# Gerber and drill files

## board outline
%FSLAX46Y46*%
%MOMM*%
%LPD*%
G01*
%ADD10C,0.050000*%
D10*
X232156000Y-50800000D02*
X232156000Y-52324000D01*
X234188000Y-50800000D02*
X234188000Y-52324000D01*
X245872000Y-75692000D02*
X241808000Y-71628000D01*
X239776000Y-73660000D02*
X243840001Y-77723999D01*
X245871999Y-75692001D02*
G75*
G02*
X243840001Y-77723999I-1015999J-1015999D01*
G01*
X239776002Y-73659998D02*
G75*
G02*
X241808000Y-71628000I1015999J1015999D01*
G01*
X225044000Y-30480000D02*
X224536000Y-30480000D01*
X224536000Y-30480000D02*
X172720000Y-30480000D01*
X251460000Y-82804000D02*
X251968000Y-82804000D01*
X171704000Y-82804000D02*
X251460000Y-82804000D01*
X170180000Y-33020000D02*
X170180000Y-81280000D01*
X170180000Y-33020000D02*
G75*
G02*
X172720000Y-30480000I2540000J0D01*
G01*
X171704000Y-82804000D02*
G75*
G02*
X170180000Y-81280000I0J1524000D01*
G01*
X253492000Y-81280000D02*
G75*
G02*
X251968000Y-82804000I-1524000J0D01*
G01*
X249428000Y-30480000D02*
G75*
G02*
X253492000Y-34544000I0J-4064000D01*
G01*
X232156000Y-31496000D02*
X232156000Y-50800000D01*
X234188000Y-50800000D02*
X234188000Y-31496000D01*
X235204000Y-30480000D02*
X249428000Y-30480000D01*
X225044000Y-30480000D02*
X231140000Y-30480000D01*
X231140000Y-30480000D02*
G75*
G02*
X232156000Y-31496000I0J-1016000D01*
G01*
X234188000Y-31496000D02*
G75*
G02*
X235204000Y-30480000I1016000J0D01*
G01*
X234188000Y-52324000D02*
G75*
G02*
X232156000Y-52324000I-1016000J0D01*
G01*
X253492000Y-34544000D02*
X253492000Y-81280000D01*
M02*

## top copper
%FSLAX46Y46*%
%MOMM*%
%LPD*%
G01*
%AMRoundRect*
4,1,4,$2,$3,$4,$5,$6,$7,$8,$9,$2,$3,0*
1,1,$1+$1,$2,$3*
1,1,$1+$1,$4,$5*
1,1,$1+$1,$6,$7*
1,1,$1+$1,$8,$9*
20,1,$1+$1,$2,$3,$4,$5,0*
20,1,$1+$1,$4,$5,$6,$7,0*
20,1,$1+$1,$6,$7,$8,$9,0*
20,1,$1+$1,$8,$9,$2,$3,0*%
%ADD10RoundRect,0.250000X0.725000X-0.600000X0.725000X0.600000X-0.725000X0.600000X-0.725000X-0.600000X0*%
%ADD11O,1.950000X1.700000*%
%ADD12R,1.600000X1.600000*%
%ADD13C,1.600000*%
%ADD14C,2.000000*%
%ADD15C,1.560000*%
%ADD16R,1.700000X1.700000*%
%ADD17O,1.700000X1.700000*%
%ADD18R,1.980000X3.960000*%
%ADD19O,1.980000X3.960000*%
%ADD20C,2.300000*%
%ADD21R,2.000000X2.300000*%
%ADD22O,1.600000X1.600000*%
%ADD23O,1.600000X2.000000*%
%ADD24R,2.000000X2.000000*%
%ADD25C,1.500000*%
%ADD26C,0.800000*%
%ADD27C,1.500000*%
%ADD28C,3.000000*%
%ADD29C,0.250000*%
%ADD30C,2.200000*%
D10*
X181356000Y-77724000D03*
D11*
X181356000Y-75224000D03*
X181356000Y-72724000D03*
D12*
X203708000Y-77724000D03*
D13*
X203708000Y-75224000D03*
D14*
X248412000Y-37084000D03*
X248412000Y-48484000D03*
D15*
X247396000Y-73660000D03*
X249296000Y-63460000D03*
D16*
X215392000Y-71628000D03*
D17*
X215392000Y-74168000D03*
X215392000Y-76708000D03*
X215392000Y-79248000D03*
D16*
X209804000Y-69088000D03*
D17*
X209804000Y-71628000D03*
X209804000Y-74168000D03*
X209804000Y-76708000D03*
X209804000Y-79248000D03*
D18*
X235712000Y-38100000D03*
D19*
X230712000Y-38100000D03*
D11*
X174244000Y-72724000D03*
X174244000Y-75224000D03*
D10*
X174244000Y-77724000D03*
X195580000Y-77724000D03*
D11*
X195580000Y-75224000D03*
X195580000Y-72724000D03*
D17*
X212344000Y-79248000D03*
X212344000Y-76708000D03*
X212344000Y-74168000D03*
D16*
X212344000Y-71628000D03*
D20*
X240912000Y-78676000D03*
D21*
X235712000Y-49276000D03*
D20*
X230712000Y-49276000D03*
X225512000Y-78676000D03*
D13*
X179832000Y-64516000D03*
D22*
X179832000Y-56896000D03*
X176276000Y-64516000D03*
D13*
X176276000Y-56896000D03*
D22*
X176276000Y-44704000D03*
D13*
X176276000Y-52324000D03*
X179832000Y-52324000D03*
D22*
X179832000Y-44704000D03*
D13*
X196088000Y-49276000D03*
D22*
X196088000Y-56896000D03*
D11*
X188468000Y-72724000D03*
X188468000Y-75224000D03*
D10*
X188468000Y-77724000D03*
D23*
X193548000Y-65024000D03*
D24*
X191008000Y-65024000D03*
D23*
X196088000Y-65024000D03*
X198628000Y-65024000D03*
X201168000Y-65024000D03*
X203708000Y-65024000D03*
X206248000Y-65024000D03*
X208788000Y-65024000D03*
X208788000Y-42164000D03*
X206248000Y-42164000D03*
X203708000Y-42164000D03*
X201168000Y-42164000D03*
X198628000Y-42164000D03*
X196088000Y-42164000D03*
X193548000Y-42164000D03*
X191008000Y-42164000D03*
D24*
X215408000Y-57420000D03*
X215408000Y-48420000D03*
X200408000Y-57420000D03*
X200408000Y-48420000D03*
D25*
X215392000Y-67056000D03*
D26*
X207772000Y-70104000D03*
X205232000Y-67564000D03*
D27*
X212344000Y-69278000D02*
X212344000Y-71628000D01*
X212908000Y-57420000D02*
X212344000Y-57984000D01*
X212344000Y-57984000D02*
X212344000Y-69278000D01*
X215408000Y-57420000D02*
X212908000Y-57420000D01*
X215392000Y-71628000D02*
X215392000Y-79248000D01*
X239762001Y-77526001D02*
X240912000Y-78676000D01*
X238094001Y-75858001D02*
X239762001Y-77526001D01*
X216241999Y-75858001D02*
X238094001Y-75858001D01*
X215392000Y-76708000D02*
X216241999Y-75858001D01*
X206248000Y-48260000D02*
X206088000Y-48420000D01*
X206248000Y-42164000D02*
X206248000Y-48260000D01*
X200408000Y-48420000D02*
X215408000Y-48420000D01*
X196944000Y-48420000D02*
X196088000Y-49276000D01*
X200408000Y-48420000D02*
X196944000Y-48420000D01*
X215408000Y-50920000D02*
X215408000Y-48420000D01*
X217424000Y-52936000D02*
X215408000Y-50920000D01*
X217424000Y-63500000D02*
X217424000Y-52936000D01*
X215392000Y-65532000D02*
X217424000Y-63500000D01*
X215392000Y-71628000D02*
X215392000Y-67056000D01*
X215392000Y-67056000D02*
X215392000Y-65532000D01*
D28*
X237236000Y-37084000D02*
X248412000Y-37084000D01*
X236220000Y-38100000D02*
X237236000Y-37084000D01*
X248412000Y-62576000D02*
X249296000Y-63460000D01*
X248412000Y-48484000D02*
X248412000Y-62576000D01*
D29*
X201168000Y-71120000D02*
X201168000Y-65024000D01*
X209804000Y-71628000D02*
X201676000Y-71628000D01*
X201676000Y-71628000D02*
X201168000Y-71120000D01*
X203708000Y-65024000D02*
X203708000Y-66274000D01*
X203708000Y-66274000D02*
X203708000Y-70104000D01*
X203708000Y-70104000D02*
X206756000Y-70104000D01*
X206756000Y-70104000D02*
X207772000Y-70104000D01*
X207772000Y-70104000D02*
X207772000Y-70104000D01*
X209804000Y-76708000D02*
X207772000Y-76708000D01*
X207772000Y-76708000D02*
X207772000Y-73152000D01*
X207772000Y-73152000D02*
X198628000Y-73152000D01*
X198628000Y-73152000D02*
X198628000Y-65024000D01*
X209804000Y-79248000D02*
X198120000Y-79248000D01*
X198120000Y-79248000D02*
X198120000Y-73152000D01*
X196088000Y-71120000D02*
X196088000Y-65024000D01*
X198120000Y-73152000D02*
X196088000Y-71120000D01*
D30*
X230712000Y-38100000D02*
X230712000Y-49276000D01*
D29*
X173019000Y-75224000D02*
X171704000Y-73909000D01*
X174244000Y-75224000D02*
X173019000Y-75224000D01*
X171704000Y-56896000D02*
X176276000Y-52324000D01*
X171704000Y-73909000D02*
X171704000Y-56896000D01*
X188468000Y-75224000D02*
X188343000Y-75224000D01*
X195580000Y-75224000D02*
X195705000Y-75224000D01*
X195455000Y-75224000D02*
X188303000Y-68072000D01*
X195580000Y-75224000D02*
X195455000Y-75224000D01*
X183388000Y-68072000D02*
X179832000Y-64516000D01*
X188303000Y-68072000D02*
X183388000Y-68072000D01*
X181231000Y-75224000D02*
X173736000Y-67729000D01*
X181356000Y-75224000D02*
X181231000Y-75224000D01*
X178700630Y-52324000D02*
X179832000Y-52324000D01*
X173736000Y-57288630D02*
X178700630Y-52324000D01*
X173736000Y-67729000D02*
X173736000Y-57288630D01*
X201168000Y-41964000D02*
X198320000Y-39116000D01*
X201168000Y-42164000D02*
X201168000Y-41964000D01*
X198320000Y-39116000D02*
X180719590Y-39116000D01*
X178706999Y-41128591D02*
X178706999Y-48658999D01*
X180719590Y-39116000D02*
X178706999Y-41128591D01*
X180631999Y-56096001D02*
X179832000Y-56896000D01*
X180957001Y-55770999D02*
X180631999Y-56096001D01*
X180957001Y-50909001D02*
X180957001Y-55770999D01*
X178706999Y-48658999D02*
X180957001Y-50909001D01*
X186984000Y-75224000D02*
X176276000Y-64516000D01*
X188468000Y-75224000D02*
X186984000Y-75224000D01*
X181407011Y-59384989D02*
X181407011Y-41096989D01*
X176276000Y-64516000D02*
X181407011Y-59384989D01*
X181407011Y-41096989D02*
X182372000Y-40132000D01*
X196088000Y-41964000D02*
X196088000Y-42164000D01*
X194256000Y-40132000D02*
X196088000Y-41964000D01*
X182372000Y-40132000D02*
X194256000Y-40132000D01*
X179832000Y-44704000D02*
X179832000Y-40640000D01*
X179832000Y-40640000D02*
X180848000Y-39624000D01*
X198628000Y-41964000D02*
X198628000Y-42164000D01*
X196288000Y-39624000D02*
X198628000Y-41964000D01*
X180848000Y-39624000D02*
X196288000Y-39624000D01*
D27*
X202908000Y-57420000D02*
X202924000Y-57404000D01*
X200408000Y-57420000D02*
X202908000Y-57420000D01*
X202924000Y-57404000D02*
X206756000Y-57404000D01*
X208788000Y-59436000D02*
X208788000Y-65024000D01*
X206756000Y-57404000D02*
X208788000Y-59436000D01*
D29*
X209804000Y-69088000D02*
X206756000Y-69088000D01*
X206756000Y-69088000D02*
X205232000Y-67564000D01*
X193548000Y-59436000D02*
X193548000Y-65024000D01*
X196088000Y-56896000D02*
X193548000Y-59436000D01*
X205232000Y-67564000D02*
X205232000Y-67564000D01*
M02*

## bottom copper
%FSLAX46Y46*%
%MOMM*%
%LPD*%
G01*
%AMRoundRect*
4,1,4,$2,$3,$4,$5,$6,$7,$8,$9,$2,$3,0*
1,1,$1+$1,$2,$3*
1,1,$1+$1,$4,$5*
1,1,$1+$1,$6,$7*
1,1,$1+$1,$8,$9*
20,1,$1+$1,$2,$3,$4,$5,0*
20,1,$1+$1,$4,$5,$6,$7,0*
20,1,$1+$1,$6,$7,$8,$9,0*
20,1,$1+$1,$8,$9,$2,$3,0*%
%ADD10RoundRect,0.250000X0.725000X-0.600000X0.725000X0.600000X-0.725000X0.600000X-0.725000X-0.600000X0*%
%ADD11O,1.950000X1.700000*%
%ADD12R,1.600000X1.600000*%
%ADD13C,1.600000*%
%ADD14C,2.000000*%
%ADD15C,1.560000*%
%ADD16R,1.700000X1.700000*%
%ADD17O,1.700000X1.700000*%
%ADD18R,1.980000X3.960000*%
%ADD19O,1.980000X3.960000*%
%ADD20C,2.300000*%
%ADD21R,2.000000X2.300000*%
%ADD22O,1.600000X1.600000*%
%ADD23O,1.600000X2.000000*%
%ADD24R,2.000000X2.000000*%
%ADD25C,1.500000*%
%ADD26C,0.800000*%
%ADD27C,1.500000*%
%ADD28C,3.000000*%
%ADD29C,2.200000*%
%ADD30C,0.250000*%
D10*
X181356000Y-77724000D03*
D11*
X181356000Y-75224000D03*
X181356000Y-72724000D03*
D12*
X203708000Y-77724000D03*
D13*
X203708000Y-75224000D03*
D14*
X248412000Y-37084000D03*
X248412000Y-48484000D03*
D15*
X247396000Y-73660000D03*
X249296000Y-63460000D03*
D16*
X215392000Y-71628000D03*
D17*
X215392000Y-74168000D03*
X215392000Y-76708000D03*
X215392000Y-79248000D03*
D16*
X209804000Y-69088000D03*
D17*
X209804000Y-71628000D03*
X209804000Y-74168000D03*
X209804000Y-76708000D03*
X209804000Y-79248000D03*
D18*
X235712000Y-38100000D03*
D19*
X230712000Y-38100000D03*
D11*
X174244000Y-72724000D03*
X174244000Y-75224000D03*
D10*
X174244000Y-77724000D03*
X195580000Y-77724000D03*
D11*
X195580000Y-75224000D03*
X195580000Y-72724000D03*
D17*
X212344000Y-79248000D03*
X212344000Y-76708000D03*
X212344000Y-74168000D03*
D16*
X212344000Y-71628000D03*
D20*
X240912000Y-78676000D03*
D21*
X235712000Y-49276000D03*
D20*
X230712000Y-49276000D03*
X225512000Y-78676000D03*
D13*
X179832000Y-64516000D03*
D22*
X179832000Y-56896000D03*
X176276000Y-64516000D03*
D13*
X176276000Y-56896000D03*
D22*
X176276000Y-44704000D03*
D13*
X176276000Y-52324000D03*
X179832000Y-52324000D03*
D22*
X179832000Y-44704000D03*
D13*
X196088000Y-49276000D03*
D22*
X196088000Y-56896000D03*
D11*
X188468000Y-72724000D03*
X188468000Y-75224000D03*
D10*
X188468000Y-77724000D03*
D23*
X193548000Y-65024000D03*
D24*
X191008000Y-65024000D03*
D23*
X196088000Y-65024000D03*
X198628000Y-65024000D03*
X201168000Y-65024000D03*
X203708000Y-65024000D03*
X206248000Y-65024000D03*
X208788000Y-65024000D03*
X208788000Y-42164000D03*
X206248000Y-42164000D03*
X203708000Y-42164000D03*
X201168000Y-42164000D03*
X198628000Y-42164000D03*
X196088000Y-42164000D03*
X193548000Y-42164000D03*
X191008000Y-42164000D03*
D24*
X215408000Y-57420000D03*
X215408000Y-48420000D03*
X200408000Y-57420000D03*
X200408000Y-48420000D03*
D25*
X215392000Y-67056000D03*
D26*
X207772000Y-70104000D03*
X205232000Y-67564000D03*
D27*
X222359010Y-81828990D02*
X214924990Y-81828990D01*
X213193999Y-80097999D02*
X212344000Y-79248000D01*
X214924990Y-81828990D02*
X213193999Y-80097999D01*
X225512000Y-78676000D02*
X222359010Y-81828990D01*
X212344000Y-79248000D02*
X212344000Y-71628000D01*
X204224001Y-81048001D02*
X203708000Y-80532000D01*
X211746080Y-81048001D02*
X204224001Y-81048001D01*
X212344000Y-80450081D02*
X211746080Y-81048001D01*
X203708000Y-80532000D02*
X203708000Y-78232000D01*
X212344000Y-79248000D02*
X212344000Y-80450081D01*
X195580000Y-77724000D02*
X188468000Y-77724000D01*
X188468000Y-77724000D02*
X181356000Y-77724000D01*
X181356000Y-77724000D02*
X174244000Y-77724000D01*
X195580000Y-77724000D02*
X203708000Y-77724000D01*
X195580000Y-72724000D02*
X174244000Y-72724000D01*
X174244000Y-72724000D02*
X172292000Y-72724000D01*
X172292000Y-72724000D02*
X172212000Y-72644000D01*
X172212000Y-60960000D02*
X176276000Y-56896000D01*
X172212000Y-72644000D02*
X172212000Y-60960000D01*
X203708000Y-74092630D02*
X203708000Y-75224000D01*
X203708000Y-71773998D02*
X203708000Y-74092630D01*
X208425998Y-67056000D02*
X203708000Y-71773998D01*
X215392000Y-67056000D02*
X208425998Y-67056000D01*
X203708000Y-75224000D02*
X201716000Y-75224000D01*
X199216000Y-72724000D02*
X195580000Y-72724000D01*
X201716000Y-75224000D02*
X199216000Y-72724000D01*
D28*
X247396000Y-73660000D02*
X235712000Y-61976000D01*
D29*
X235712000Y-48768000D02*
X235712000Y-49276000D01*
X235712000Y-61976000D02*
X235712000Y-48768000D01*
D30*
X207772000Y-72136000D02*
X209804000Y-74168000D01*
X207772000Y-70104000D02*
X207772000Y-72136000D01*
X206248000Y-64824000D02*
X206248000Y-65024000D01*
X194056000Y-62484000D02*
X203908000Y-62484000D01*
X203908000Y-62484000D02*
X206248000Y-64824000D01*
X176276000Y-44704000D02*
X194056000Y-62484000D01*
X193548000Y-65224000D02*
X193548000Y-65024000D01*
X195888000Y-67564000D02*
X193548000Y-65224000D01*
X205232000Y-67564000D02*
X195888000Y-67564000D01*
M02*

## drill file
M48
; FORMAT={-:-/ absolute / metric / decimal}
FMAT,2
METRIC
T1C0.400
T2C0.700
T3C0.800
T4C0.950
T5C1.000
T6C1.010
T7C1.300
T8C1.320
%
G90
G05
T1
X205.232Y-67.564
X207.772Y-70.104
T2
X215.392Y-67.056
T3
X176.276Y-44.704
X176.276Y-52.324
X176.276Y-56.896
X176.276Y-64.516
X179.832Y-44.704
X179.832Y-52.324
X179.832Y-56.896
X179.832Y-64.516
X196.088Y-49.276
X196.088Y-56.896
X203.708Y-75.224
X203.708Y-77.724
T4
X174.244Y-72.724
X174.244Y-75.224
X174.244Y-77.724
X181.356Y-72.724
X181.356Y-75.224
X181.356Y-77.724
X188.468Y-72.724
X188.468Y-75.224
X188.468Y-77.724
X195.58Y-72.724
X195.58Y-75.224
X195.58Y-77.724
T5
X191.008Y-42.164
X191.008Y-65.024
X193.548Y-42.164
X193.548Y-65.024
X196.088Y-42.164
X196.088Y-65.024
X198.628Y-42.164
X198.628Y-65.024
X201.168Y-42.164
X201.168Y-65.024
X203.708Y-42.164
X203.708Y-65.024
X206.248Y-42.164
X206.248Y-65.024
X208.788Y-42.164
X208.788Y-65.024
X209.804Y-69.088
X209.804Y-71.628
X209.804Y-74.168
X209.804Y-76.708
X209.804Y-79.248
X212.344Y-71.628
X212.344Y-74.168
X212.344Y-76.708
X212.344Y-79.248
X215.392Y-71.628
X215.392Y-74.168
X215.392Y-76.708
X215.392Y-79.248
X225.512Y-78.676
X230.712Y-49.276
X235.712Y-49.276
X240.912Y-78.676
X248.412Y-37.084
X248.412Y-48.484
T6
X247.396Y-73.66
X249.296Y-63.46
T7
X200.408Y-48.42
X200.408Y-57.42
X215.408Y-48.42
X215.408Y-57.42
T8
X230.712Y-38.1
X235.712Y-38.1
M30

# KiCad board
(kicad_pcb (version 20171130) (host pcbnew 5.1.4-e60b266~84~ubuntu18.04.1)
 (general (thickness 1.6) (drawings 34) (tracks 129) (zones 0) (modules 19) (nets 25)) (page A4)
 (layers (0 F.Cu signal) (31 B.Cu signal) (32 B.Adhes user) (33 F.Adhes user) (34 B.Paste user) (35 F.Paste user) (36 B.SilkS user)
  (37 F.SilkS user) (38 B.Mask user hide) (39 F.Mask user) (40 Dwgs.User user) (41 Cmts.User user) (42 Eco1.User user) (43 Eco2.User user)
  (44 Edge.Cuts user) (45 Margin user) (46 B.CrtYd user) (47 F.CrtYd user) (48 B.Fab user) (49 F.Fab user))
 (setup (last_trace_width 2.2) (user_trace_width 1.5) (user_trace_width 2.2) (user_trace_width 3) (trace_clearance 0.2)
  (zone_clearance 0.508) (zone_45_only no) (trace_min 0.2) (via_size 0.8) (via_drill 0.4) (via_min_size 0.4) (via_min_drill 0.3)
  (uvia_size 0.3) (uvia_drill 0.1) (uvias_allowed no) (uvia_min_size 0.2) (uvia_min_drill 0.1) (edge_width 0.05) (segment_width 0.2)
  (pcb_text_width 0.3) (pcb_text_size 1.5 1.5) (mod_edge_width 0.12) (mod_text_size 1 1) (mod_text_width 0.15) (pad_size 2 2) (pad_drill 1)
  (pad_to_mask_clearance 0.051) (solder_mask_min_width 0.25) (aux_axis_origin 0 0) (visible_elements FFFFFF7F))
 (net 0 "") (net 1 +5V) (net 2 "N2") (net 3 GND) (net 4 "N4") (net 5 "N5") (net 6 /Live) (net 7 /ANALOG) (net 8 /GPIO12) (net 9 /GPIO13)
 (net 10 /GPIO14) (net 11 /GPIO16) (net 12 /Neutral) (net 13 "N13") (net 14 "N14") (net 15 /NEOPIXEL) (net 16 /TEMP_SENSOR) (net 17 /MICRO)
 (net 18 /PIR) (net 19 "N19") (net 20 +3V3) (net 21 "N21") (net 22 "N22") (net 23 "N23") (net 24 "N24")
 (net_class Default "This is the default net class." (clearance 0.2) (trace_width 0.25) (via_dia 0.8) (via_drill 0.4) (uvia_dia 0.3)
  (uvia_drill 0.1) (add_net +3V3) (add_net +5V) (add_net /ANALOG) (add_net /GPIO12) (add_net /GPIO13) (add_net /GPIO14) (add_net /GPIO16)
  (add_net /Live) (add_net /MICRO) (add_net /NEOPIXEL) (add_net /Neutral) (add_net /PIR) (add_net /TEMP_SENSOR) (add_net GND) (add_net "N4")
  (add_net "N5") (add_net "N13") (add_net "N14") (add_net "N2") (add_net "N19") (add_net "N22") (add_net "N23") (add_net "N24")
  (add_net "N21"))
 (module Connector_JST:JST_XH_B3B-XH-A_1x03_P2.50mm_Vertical (layer F.Cu) (at 181.356 77.724 90)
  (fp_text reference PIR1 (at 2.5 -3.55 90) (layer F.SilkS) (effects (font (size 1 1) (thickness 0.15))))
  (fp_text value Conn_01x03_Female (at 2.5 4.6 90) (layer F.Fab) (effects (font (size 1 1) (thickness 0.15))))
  (pad 1 thru_hole roundrect (at 0 0 90) (size 1.7 1.95) (drill 0.95) (layers *.Cu *.Mask) (roundrect_rratio 0.147059) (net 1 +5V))
  (pad 2 thru_hole oval (at 2.5 0 90) (size 1.7 1.95) (drill 0.95) (layers *.Cu *.Mask) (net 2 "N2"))
  (pad 3 thru_hole oval (at 5 0 90) (size 1.7 1.95) (drill 0.95) (layers *.Cu *.Mask) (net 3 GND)))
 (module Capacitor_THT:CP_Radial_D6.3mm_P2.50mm (layer F.Cu) (at 203.708 77.724 90)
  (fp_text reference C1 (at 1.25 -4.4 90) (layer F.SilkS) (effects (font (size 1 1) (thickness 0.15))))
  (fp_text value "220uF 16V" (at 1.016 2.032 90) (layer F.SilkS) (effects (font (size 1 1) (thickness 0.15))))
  (pad 1 thru_hole rect (at 0 0 90) (size 1.6 1.6) (drill 0.8) (layers *.Cu *.Mask) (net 1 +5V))
  (pad 2 thru_hole circle (at 2.5 0 90) (size 1.6 1.6) (drill 0.8) (layers *.Cu *.Mask) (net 3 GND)))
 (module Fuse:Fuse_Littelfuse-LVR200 (layer F.Cu) (at 248.412 37.084 270)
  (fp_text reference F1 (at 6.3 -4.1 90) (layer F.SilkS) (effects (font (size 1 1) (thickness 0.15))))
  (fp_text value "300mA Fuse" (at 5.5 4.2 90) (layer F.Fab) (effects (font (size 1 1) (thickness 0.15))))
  (pad 1 thru_hole circle (at 0 0 270) (size 2 2) (drill 1) (layers *.Cu *.Mask) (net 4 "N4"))
  (pad 2 thru_hole circle (at 11.4 0 270) (size 2 2) (drill 1) (layers *.Cu *.Mask) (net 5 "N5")))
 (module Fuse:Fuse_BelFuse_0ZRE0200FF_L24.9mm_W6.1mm (layer F.Cu) (at 247.396 73.66 90)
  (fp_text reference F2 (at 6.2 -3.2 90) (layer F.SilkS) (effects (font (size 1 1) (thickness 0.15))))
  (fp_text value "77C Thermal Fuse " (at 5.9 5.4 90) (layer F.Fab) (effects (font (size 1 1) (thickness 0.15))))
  (pad 1 thru_hole circle (at 0 0 90) (size 1.56 1.56) (drill 1.01) (layers *.Cu *.Mask) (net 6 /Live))
  (pad 2 thru_hole circle (at 10.2 1.9 90) (size 1.56 1.56) (drill 1.01) (layers *.Cu *.Mask) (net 5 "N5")))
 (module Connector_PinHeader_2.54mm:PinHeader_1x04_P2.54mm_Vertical (layer F.Cu) (at 215.392 71.628)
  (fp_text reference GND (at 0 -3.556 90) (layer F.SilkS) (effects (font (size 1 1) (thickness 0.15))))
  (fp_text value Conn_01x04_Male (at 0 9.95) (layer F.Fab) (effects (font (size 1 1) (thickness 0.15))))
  (pad 1 thru_hole rect (at 0 0) (size 1.7 1.7) (drill 1) (layers *.Cu *.Mask) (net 3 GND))
  (pad 2 thru_hole oval (at 0 2.54) (size 1.7 1.7) (drill 1) (layers *.Cu *.Mask) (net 3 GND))
  (pad 3 thru_hole oval (at 0 5.08) (size 1.7 1.7) (drill 1) (layers *.Cu *.Mask) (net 3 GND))
  (pad 4 thru_hole oval (at 0 7.62) (size 1.7 1.7) (drill 1) (layers *.Cu *.Mask) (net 3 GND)))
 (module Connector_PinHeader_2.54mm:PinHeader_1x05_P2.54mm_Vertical (layer F.Cu) (at 209.804 69.088)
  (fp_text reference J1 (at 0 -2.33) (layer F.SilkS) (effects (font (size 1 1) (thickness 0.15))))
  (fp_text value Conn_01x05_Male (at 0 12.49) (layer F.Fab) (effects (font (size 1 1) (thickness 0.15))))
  (pad 1 thru_hole rect (at 0 0) (size 1.7 1.7) (drill 1) (layers *.Cu *.Mask) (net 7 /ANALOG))
  (pad 2 thru_hole oval (at 0 2.54) (size 1.7 1.7) (drill 1) (layers *.Cu *.Mask) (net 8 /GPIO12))
  (pad 3 thru_hole oval (at 0 5.08) (size 1.7 1.7) (drill 1) (layers *.Cu *.Mask) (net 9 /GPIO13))
  (pad 4 thru_hole oval (at 0 7.62) (size 1.7 1.7) (drill 1) (layers *.Cu *.Mask) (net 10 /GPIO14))
  (pad 5 thru_hole oval (at 0 10.16) (size 1.7 1.7) (drill 1) (layers *.Cu *.Mask) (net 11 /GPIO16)))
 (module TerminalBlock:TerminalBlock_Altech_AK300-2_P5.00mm (layer F.Cu) (at 235.712 38.1 180)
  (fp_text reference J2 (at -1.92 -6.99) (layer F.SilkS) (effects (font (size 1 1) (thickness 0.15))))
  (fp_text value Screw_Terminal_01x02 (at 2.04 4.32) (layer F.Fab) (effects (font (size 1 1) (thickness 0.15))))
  (pad 1 thru_hole rect (at 0 0 180) (size 1.98 3.96) (drill 1.32) (layers *.Cu *.Mask) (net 4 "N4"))
  (pad 2 thru_hole oval (at 5 0 180) (size 1.98 3.96) (drill 1.32) (layers *.Cu *.Mask) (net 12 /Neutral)))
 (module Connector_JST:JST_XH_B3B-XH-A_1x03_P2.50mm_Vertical (layer F.Cu) (at 174.244 77.724 90)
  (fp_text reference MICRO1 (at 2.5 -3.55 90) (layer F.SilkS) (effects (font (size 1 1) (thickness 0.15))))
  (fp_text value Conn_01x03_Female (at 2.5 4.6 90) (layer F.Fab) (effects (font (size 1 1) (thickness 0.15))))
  (pad 3 thru_hole oval (at 5 0 90) (size 1.7 1.95) (drill 0.95) (layers *.Cu *.Mask) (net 3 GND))
  (pad 2 thru_hole oval (at 2.5 0 90) (size 1.7 1.95) (drill 0.95) (layers *.Cu *.Mask) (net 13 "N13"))
  (pad 1 thru_hole roundrect (at 0 0 90) (size 1.7 1.95) (drill 0.95) (layers *.Cu *.Mask) (roundrect_rratio 0.147059) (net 1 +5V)))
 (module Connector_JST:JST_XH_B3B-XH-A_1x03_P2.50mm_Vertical (layer F.Cu) (at 195.58 77.724 90)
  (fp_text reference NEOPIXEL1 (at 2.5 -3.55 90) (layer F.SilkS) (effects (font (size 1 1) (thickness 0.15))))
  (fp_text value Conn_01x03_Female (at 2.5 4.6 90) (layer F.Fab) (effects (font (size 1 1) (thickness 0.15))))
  (pad 1 thru_hole roundrect (at 0 0 90) (size 1.7 1.95) (drill 0.95) (layers *.Cu *.Mask) (roundrect_rratio 0.147059) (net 1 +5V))
  (pad 2 thru_hole oval (at 2.5 0 90) (size 1.7 1.95) (drill 0.95) (layers *.Cu *.Mask) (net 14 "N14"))
  (pad 3 thru_hole oval (at 5 0 90) (size 1.7 1.95) (drill 0.95) (layers *.Cu *.Mask) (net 3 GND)))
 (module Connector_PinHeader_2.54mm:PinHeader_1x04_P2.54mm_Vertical (layer F.Cu) (at 212.344 71.628)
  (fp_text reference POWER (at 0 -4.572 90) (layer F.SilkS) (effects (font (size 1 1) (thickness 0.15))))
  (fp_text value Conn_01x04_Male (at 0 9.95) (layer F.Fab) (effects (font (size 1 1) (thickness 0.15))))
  (pad 4 thru_hole oval (at 0 7.62) (size 1.7 1.7) (drill 1) (layers *.Cu *.Mask) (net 1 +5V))
  (pad 3 thru_hole oval (at 0 5.08) (size 1.7 1.7) (drill 1) (layers *.Cu *.Mask) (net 1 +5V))
  (pad 2 thru_hole oval (at 0 2.54) (size 1.7 1.7) (drill 1) (layers *.Cu *.Mask) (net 1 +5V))
  (pad 1 thru_hole rect (at 0 0) (size 1.7 1.7) (drill 1) (layers *.Cu *.Mask) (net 1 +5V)))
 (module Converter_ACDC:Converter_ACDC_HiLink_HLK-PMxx (layer F.Cu) (at 235.712 49.276 270)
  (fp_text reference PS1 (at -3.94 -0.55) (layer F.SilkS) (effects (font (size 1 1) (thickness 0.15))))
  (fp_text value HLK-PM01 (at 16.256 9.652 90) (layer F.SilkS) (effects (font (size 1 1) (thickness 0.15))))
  (pad 3 thru_hole circle (at 29.4 -5.2 270) (size 2.3 2.3) (drill 1) (layers *.Cu *.Mask) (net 3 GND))
  (pad 1 thru_hole rect (at 0 0 270) (size 2.3 2) (drill 1) (layers *.Cu *.Mask) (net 6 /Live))
  (pad 2 thru_hole circle (at 0 5 270) (size 2.3 2.3) (drill 1) (layers *.Cu *.Mask) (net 12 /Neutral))
  (pad 4 thru_hole circle (at 29.4 10.2 270) (size 2.3 2.3) (drill 1) (layers *.Cu *.Mask) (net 1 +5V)))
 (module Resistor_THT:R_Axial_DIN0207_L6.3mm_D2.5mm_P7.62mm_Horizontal (layer F.Cu) (at 179.832 64.516 90)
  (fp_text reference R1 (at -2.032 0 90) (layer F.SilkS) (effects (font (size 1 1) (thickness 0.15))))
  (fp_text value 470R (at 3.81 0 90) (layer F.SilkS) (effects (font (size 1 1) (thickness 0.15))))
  (pad 1 thru_hole circle (at 0 0 90) (size 1.6 1.6) (drill 0.8) (layers *.Cu *.Mask) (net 14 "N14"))
  (pad 2 thru_hole oval (at 7.62 0 90) (size 1.6 1.6) (drill 0.8) (layers *.Cu *.Mask) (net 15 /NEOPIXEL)))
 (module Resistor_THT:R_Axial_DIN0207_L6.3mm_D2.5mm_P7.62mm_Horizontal (layer F.Cu) (at 176.276 56.896 270)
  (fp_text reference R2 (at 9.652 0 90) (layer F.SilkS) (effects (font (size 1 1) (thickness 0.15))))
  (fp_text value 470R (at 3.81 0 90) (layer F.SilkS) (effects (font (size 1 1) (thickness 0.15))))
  (pad 2 thru_hole oval (at 7.62 0 270) (size 1.6 1.6) (drill 0.8) (layers *.Cu *.Mask) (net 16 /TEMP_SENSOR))
  (pad 1 thru_hole circle (at 0 0 270) (size 1.6 1.6) (drill 0.8) (layers *.Cu *.Mask) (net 3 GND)))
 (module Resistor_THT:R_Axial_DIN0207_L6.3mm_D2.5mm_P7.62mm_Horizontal (layer F.Cu) (at 176.276 52.324 90)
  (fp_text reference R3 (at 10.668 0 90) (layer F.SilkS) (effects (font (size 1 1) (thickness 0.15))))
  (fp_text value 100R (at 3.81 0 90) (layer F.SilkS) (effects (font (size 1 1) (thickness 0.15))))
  (pad 2 thru_hole oval (at 7.62 0 90) (size 1.6 1.6) (drill 0.8) (layers *.Cu *.Mask) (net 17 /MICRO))
  (pad 1 thru_hole circle (at 0 0 90) (size 1.6 1.6) (drill 0.8) (layers *.Cu *.Mask) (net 13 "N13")))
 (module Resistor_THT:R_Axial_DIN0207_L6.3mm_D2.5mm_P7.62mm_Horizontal (layer F.Cu) (at 179.832 52.324 90)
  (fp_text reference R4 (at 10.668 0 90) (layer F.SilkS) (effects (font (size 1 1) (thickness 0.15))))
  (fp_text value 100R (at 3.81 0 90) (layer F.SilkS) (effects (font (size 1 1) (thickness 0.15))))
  (pad 1 thru_hole circle (at 0 0 90) (size 1.6 1.6) (drill 0.8) (layers *.Cu *.Mask) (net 2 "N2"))
  (pad 2 thru_hole oval (at 7.62 0 90) (size 1.6 1.6) (drill 0.8) (layers *.Cu *.Mask) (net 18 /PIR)))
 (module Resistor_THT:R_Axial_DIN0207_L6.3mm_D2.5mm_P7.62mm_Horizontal (layer F.Cu) (at 196.088 49.276 270)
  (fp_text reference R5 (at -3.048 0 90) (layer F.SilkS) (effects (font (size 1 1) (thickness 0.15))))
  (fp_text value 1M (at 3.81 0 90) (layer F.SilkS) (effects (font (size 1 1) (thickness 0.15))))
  (pad 1 thru_hole circle (at 0 0 270) (size 1.6 1.6) (drill 0.8) (layers *.Cu *.Mask) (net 3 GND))
  (pad 2 thru_hole oval (at 7.62 0 270) (size 1.6 1.6) (drill 0.8) (layers *.Cu *.Mask) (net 7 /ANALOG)))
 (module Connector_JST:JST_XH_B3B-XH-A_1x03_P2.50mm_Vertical (layer F.Cu) (at 188.468 77.724 90)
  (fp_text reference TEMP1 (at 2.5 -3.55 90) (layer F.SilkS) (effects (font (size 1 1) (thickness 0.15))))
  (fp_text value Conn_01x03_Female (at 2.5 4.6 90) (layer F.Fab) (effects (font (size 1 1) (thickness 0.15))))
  (pad 3 thru_hole oval (at 5 0 90) (size 1.7 1.95) (drill 0.95) (layers *.Cu *.Mask) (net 3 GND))
  (pad 2 thru_hole oval (at 2.5 0 90) (size 1.7 1.95) (drill 0.95) (layers *.Cu *.Mask) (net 16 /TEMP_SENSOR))
  (pad 1 thru_hole roundrect (at 0 0 90) (size 1.7 1.95) (drill 0.95) (layers *.Cu *.Mask) (roundrect_rratio 0.147059) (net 1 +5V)))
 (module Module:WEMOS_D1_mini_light (layer F.Cu) (at 191.008 65.024 90)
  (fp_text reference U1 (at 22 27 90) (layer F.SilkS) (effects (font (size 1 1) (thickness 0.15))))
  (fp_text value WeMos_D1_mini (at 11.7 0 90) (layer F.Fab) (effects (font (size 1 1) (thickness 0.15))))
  (pad 2 thru_hole oval (at 0 2.54 90) (size 2 1.6) (drill 1) (layers *.Cu *.Mask) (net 7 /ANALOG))
  (pad 1 thru_hole rect (at 0 0 90) (size 2 2) (drill 1) (layers *.Cu *.Mask) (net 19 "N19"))
  (pad 3 thru_hole oval (at 0 5.08 90) (size 2 1.6) (drill 1) (layers *.Cu *.Mask) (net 11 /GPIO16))
  (pad 4 thru_hole oval (at 0 7.62 90) (size 2 1.6) (drill 1) (layers *.Cu *.Mask) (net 10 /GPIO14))
  (pad 5 thru_hole oval (at 0 10.16 90) (size 2 1.6) (drill 1) (layers *.Cu *.Mask) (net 8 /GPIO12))
  (pad 6 thru_hole oval (at 0 12.7 90) (size 2 1.6) (drill 1) (layers *.Cu *.Mask) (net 9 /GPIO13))
  (pad 7 thru_hole oval (at 0 15.24 90) (size 2 1.6) (drill 1) (layers *.Cu *.Mask) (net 17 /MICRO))
  (pad 8 thru_hole oval (at 0 17.78 90) (size 2 1.6) (drill 1) (layers *.Cu *.Mask) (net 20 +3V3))
  (pad 9 thru_hole oval (at 22.86 17.78 90) (size 2 1.6) (drill 1) (layers *.Cu *.Mask) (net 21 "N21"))
  (pad 10 thru_hole oval (at 22.86 15.24 90) (size 2 1.6) (drill 1) (layers *.Cu *.Mask) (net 3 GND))
  (pad 11 thru_hole oval (at 22.86 12.7 90) (size 2 1.6) (drill 1) (layers *.Cu *.Mask) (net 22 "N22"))
  (pad 12 thru_hole oval (at 22.86 10.16 90) (size 2 1.6) (drill 1) (layers *.Cu *.Mask) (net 15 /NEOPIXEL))
  (pad 13 thru_hole oval (at 22.86 7.62 90) (size 2 1.6) (drill 1) (layers *.Cu *.Mask) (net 18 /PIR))
  (pad 14 thru_hole oval (at 22.86 5.08 90) (size 2 1.6) (drill 1) (layers *.Cu *.Mask) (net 16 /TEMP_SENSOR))
  (pad 15 thru_hole oval (at 22.86 2.54 90) (size 2 1.6) (drill 1) (layers *.Cu *.Mask) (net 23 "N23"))
  (pad 16 thru_hole oval (at 22.86 0 90) (size 2 1.6) (drill 1) (layers *.Cu *.Mask) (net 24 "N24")))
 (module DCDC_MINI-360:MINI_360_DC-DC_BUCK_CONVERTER (layer F.Cu) (at 216.408 58.42 180)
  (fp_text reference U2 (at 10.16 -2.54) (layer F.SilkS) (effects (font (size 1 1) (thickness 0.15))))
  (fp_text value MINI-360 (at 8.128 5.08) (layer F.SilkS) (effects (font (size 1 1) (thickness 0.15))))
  (pad 1 thru_hole rect (at 1 1 180) (size 2 2) (drill 1.3) (layers *.Cu *.Mask) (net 1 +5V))
  (pad 2 thru_hole rect (at 1 10 180) (size 2 2) (drill 1.3) (layers *.Cu *.Mask) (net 3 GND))
  (pad 3 thru_hole rect (at 16 1 180) (size 2 2) (drill 1.3) (layers *.Cu *.Mask) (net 20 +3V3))
  (pad 4 thru_hole rect (at 16 10 180) (size 2 2) (drill 1.3) (layers *.Cu *.Mask) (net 3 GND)))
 (gr_line (start 232.156 50.8) (end 232.156 52.324) (layer Edge.Cuts) (width 0.05))
 (gr_line (start 234.188 50.8) (end 234.188 52.324) (layer Edge.Cuts) (width 0.05))
 (gr_line (start 245.872 75.692) (end 241.808 71.628) (layer Edge.Cuts) (width 0.05))
 (gr_line (start 239.776 73.66) (end 243.840001 77.723999) (layer Edge.Cuts) (width 0.05))
 (gr_arc (start 244.856 76.708) (end 243.840001 77.723999) (angle -180) (layer Edge.Cuts) (width 0.05))
 (gr_arc (start 240.792001 72.643999) (end 241.808 71.628) (angle -180) (layer Edge.Cuts) (width 0.05))
 (gr_line (start 225.044 30.48) (end 224.536 30.48) (layer Edge.Cuts) (width 0.05))
 (gr_line (start 224.536 30.48) (end 172.72 30.48) (layer Edge.Cuts) (width 0.05))
 (gr_line (start 251.46 82.804) (end 251.968 82.804) (layer Edge.Cuts) (width 0.05))
 (gr_line (start 171.704 82.804) (end 251.46 82.804) (layer Edge.Cuts) (width 0.05))
 (gr_line (start 170.18 33.02) (end 170.18 81.28) (layer Edge.Cuts) (width 0.05))
 (gr_arc (start 172.72 33.02) (end 172.72 30.48) (angle -90) (layer Edge.Cuts) (width 0.05))
 (gr_arc (start 171.704 81.28) (end 170.18 81.28) (angle -90) (layer Edge.Cuts) (width 0.05))
 (gr_arc (start 251.968 81.28) (end 251.968 82.804) (angle -90) (layer Edge.Cuts) (width 0.05))
 (gr_arc (start 249.428 34.544) (end 253.492 34.544) (angle -90) (layer Edge.Cuts) (width 0.05))
 (gr_line (start 232.156 31.496) (end 232.156 50.8) (layer Edge.Cuts) (width 0.05))
 (gr_line (start 234.188 50.8) (end 234.188 31.496) (layer Edge.Cuts) (width 0.05))
 (gr_line (start 235.204 30.48) (end 249.428 30.48) (layer Edge.Cuts) (width 0.05))
 (gr_line (start 225.044 30.48) (end 231.14 30.48) (layer Edge.Cuts) (width 0.05))
 (gr_arc (start 231.14 31.496) (end 232.156 31.496) (angle -90) (layer Edge.Cuts) (width 0.05))
 (gr_arc (start 235.204 31.496) (end 235.204 30.48) (angle -90) (layer Edge.Cuts) (width 0.05))
 (gr_arc (start 233.172 52.324) (end 232.156 52.324) (angle -180) (layer Edge.Cuts) (width 0.05))
 (gr_line (start 253.492 34.544) (end 253.492 81.28) (layer Edge.Cuts) (width 0.05))
 (segment (start 222.35901 81.82899) (end 214.92499 81.82899) (width 1.5) (layer B.Cu) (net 1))
 (segment (start 213.193999 80.097999) (end 212.344 79.248) (width 1.5) (layer B.Cu) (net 1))
 (segment (start 214.92499 81.82899) (end 213.193999 80.097999) (width 1.5) (layer B.Cu) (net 1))
 (segment (start 225.512 78.676) (end 222.35901 81.82899) (width 1.5) (layer B.Cu) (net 1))
 (segment (start 212.344 79.248) (end 212.344 71.628) (width 1.5) (layer B.Cu) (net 1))
 (segment (start 204.224001 81.048001) (end 203.708 80.532) (width 1.5) (layer B.Cu) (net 1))
 (segment (start 211.74608 81.048001) (end 204.224001 81.048001) (width 1.5) (layer B.Cu) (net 1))
 (segment (start 212.344 80.450081) (end 211.74608 81.048001) (width 1.5) (layer B.Cu) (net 1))
 (segment (start 203.708 80.532) (end 203.708 78.232) (width 1.5) (layer B.Cu) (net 1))
 (segment (start 212.344 79.248) (end 212.344 80.450081) (width 1.5) (layer B.Cu) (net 1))
 (segment (start 195.58 77.724) (end 188.468 77.724) (width 1.5) (layer B.Cu) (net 1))
 (segment (start 188.468 77.724) (end 181.356 77.724) (width 1.5) (layer B.Cu) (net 1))
 (segment (start 181.356 77.724) (end 174.244 77.724) (width 1.5) (layer B.Cu) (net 1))
 (segment (start 195.58 77.724) (end 203.708 77.724) (width 1.5) (layer B.Cu) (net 1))
 (segment (start 212.344 69.278) (end 212.344 71.628) (width 1.5) (layer F.Cu) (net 1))
 (segment (start 212.908 57.42) (end 212.344 57.984) (width 1.5) (layer F.Cu) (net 1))
 (segment (start 212.344 57.984) (end 212.344 69.278) (width 1.5) (layer F.Cu) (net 1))
 (segment (start 215.408 57.42) (end 212.908 57.42) (width 1.5) (layer F.Cu) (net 1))
 (segment (start 215.392 71.628) (end 215.392 79.248) (width 1.5) (layer F.Cu) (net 3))
 (segment (start 239.762001 77.526001) (end 240.912 78.676) (width 1.5) (layer F.Cu) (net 3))
 (segment (start 238.094001 75.858001) (end 239.762001 77.526001) (width 1.5) (layer F.Cu) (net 3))
 (segment (start 216.241999 75.858001) (end 238.094001 75.858001) (width 1.5) (layer F.Cu) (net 3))
 (segment (start 215.392 76.708) (end 216.241999 75.858001) (width 1.5) (layer F.Cu) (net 3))
 (segment (start 206.248 48.26) (end 206.088 48.42) (width 1.5) (layer F.Cu) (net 3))
 (segment (start 206.248 42.164) (end 206.248 48.26) (width 1.5) (layer F.Cu) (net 3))
 (segment (start 200.408 48.42) (end 215.408 48.42) (width 1.5) (layer F.Cu) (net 3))
 (segment (start 196.944 48.42) (end 196.088 49.276) (width 1.5) (layer F.Cu) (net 3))
 (segment (start 200.408 48.42) (end 196.944 48.42) (width 1.5) (layer F.Cu) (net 3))
 (segment (start 195.58 72.724) (end 174.244 72.724) (width 1.5) (layer B.Cu) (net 3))
 (segment (start 174.244 72.724) (end 172.292 72.724) (width 1.5) (layer B.Cu) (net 3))
 (segment (start 172.292 72.724) (end 172.212 72.644) (width 1.5) (layer B.Cu) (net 3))
 (segment (start 172.212 60.96) (end 176.276 56.896) (width 1.5) (layer B.Cu) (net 3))
 (segment (start 172.212 72.644) (end 172.212 60.96) (width 1.5) (layer B.Cu) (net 3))
 (segment (start 215.408 50.92) (end 215.408 48.42) (width 1.5) (layer F.Cu) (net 3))
 (segment (start 217.424 52.936) (end 215.408 50.92) (width 1.5) (layer F.Cu) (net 3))
 (segment (start 217.424 63.5) (end 217.424 52.936) (width 1.5) (layer F.Cu) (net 3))
 (segment (start 215.392 65.532) (end 217.424 63.5) (width 1.5) (layer F.Cu) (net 3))
 (segment (start 215.392 71.628) (end 215.392 67.056) (width 1.5) (layer F.Cu) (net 3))
 (segment (start 215.392 67.056) (end 215.392 65.532) (width 1.5) (layer F.Cu) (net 3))
 (via (at 215.392 67.056) (size 1.5) (drill 0.7) (layers F.Cu B.Cu) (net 3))
 (segment (start 203.708 74.09263) (end 203.708 75.224) (width 1.5) (layer B.Cu) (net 3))
 (segment (start 203.708 71.773998) (end 203.708 74.09263) (width 1.5) (layer B.Cu) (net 3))
 (segment (start 208.425998 67.056) (end 203.708 71.773998) (width 1.5) (layer B.Cu) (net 3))
 (segment (start 215.392 67.056) (end 208.425998 67.056) (width 1.5) (layer B.Cu) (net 3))
 (segment (start 203.708 75.224) (end 201.716 75.224) (width 1.5) (layer B.Cu) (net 3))
 (segment (start 199.216 72.724) (end 195.58 72.724) (width 1.5) (layer B.Cu) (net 3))
 (segment (start 201.716 75.224) (end 199.216 72.724) (width 1.5) (layer B.Cu) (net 3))
 (segment (start 237.236 37.084) (end 248.412 37.084) (width 3) (layer F.Cu) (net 4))
 (segment (start 236.22 38.1) (end 237.236 37.084) (width 3) (layer F.Cu) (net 4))
 (segment (start 248.412 62.576) (end 249.296 63.46) (width 3) (layer F.Cu) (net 5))
 (segment (start 248.412 48.484) (end 248.412 62.576) (width 3) (layer F.Cu) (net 5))
 (segment (start 247.396 73.66) (end 235.712 61.976) (width 3) (layer B.Cu) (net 6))
 (segment (start 235.712 48.768) (end 235.712 49.276) (width 2.2) (layer B.Cu) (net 6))
 (segment (start 235.712 61.976) (end 235.712 48.768) (width 2.2) (layer B.Cu) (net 6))
 (segment (start 201.168 71.12) (end 201.168 65.024) (width 0.25) (layer F.Cu) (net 8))
 (segment (start 209.804 71.628) (end 201.676 71.628) (width 0.25) (layer F.Cu) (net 8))
 (segment (start 201.676 71.628) (end 201.168 71.12) (width 0.25) (layer F.Cu) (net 8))
 (segment (start 203.708 65.024) (end 203.708 66.274) (width 0.25) (layer F.Cu) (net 9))
 (segment (start 203.708 66.274) (end 203.708 70.104) (width 0.25) (layer F.Cu) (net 9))
 (segment (start 203.708 70.104) (end 206.756 70.104) (width 0.25) (layer F.Cu) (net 9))
 (segment (start 206.756 70.104) (end 207.772 70.104) (width 0.25) (layer F.Cu) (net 9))
 (segment (start 207.772 70.104) (end 207.772 70.104) (width 0.25) (layer F.Cu) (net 9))
 (via (at 207.772 70.104) (size 0.8) (drill 0.4) (layers F.Cu B.Cu) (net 9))
 (segment (start 207.772 72.136) (end 209.804 74.168) (width 0.25) (layer B.Cu) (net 9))
 (segment (start 207.772 70.104) (end 207.772 72.136) (width 0.25) (layer B.Cu) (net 9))
 (segment (start 209.804 76.708) (end 207.772 76.708) (width 0.25) (layer F.Cu) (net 10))
 (segment (start 207.772 76.708) (end 207.772 73.152) (width 0.25) (layer F.Cu) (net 10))
 (segment (start 207.772 73.152) (end 198.628 73.152) (width 0.25) (layer F.Cu) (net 10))
 (segment (start 198.628 73.152) (end 198.628 65.024) (width 0.25) (layer F.Cu) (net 10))
 (segment (start 209.804 79.248) (end 198.12 79.248) (width 0.25) (layer F.Cu) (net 11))
 (segment (start 198.12 79.248) (end 198.12 73.152) (width 0.25) (layer F.Cu) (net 11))
 (segment (start 196.088 71.12) (end 196.088 65.024) (width 0.25) (layer F.Cu) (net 11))
 (segment (start 198.12 73.152) (end 196.088 71.12) (width 0.25) (layer F.Cu) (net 11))
 (segment (start 230.712 38.1) (end 230.712 49.276) (width 2.2) (layer F.Cu) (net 12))
 (segment (start 173.019 75.224) (end 171.704 73.909) (width 0.25) (layer F.Cu) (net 13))
 (segment (start 174.244 75.224) (end 173.019 75.224) (width 0.25) (layer F.Cu) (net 13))
 (segment (start 171.704 56.896) (end 176.276 52.324) (width 0.25) (layer F.Cu) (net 13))
 (segment (start 171.704 73.909) (end 171.704 56.896) (width 0.25) (layer F.Cu) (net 13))
 (segment (start 188.468 75.224) (end 188.343 75.224) (width 0.25) (layer F.Cu) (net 16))
 (segment (start 195.58 75.224) (end 195.705 75.224) (width 0.25) (layer F.Cu) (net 14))
 (segment (start 195.455 75.224) (end 188.303 68.072) (width 0.25) (layer F.Cu) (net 14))
 (segment (start 195.58 75.224) (end 195.455 75.224) (width 0.25) (layer F.Cu) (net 14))
 (segment (start 183.388 68.072) (end 179.832 64.516) (width 0.25) (layer F.Cu) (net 14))
 (segment (start 188.303 68.072) (end 183.388 68.072) (width 0.25) (layer F.Cu) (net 14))
 (segment (start 181.231 75.224) (end 173.736 67.729) (width 0.25) (layer F.Cu) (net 2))
 (segment (start 181.356 75.224) (end 181.231 75.224) (width 0.25) (layer F.Cu) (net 2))
 (segment (start 178.70063 52.324) (end 179.832 52.324) (width 0.25) (layer F.Cu) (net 2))
 (segment (start 173.736 57.28863) (end 178.70063 52.324) (width 0.25) (layer F.Cu) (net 2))
 (segment (start 173.736 67.729) (end 173.736 57.28863) (width 0.25) (layer F.Cu) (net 2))
 (segment (start 201.168 41.964) (end 198.32 39.116) (width 0.25) (layer F.Cu) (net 15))
 (segment (start 201.168 42.164) (end 201.168 41.964) (width 0.25) (layer F.Cu) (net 15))
 (segment (start 198.32 39.116) (end 180.71959 39.116) (width 0.25) (layer F.Cu) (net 15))
 (segment (start 178.706999 41.128591) (end 178.706999 48.658999) (width 0.25) (layer F.Cu) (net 15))
 (segment (start 180.71959 39.116) (end 178.706999 41.128591) (width 0.25) (layer F.Cu) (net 15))
 (segment (start 180.631999 56.096001) (end 179.832 56.896) (width 0.25) (layer F.Cu) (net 15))
 (segment (start 180.957001 55.770999) (end 180.631999 56.096001) (width 0.25) (layer F.Cu) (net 15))
 (segment (start 180.957001 50.909001) (end 180.957001 55.770999) (width 0.25) (layer F.Cu) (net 15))
 (segment (start 178.706999 48.658999) (end 180.957001 50.909001) (width 0.25) (layer F.Cu) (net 15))
 (segment (start 186.984 75.224) (end 176.276 64.516) (width 0.25) (layer F.Cu) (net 16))
 (segment (start 188.468 75.224) (end 186.984 75.224) (width 0.25) (layer F.Cu) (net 16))
 (segment (start 181.407011 59.384989) (end 181.407011 41.096989) (width 0.25) (layer F.Cu) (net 16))
 (segment (start 176.276 64.516) (end 181.407011 59.384989) (width 0.25) (layer F.Cu) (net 16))
 (segment (start 181.407011 41.096989) (end 182.372 40.132) (width 0.25) (layer F.Cu) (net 16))
 (segment (start 196.088 41.964) (end 196.088 42.164) (width 0.25) (layer F.Cu) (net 16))
 (segment (start 194.256 40.132) (end 196.088 41.964) (width 0.25) (layer F.Cu) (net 16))
 (segment (start 182.372 40.132) (end 194.256 40.132) (width 0.25) (layer F.Cu) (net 16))
 (segment (start 206.248 64.824) (end 206.248 65.024) (width 0.25) (layer B.Cu) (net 17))
 (segment (start 194.056 62.484) (end 203.908 62.484) (width 0.25) (layer B.Cu) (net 17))
 (segment (start 203.908 62.484) (end 206.248 64.824) (width 0.25) (layer B.Cu) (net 17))
 (segment (start 176.276 44.704) (end 194.056 62.484) (width 0.25) (layer B.Cu) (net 17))
 (segment (start 179.832 44.704) (end 179.832 40.64) (width 0.25) (layer F.Cu) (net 18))
 (segment (start 179.832 40.64) (end 180.848 39.624) (width 0.25) (layer F.Cu) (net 18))
 (segment (start 198.628 41.964) (end 198.628 42.164) (width 0.25) (layer F.Cu) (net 18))
 (segment (start 196.288 39.624) (end 198.628 41.964) (width 0.25) (layer F.Cu) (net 18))
 (segment (start 180.848 39.624) (end 196.288 39.624) (width 0.25) (layer F.Cu) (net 18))
 (segment (start 202.908 57.42) (end 202.924 57.404) (width 1.5) (layer F.Cu) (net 20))
 (segment (start 200.408 57.42) (end 202.908 57.42) (width 1.5) (layer F.Cu) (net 20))
 (segment (start 202.924 57.404) (end 206.756 57.404) (width 1.5) (layer F.Cu) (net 20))
 (segment (start 208.788 59.436) (end 208.788 65.024) (width 1.5) (layer F.Cu) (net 20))
 (segment (start 206.756 57.404) (end 208.788 59.436) (width 1.5) (layer F.Cu) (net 20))
 (segment (start 209.804 69.088) (end 206.756 69.088) (width 0.25) (layer F.Cu) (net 7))
 (segment (start 206.756 69.088) (end 205.232 67.564) (width 0.25) (layer F.Cu) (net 7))
 (segment (start 193.548 59.436) (end 193.548 65.024) (width 0.25) (layer F.Cu) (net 7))
 (segment (start 196.088 56.896) (end 193.548 59.436) (width 0.25) (layer F.Cu) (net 7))
 (segment (start 205.232 67.564) (end 205.232 67.564) (width 0.25) (layer F.Cu) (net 7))
 (via (at 205.232 67.564) (size 0.8) (drill 0.4) (layers F.Cu B.Cu) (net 7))
 (segment (start 193.548 65.224) (end 193.548 65.024) (width 0.25) (layer B.Cu) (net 7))
 (segment (start 195.888 67.564) (end 193.548 65.224) (width 0.25) (layer B.Cu) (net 7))
 (segment (start 205.232 67.564) (end 195.888 67.564) (width 0.25) (layer B.Cu) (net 7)))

